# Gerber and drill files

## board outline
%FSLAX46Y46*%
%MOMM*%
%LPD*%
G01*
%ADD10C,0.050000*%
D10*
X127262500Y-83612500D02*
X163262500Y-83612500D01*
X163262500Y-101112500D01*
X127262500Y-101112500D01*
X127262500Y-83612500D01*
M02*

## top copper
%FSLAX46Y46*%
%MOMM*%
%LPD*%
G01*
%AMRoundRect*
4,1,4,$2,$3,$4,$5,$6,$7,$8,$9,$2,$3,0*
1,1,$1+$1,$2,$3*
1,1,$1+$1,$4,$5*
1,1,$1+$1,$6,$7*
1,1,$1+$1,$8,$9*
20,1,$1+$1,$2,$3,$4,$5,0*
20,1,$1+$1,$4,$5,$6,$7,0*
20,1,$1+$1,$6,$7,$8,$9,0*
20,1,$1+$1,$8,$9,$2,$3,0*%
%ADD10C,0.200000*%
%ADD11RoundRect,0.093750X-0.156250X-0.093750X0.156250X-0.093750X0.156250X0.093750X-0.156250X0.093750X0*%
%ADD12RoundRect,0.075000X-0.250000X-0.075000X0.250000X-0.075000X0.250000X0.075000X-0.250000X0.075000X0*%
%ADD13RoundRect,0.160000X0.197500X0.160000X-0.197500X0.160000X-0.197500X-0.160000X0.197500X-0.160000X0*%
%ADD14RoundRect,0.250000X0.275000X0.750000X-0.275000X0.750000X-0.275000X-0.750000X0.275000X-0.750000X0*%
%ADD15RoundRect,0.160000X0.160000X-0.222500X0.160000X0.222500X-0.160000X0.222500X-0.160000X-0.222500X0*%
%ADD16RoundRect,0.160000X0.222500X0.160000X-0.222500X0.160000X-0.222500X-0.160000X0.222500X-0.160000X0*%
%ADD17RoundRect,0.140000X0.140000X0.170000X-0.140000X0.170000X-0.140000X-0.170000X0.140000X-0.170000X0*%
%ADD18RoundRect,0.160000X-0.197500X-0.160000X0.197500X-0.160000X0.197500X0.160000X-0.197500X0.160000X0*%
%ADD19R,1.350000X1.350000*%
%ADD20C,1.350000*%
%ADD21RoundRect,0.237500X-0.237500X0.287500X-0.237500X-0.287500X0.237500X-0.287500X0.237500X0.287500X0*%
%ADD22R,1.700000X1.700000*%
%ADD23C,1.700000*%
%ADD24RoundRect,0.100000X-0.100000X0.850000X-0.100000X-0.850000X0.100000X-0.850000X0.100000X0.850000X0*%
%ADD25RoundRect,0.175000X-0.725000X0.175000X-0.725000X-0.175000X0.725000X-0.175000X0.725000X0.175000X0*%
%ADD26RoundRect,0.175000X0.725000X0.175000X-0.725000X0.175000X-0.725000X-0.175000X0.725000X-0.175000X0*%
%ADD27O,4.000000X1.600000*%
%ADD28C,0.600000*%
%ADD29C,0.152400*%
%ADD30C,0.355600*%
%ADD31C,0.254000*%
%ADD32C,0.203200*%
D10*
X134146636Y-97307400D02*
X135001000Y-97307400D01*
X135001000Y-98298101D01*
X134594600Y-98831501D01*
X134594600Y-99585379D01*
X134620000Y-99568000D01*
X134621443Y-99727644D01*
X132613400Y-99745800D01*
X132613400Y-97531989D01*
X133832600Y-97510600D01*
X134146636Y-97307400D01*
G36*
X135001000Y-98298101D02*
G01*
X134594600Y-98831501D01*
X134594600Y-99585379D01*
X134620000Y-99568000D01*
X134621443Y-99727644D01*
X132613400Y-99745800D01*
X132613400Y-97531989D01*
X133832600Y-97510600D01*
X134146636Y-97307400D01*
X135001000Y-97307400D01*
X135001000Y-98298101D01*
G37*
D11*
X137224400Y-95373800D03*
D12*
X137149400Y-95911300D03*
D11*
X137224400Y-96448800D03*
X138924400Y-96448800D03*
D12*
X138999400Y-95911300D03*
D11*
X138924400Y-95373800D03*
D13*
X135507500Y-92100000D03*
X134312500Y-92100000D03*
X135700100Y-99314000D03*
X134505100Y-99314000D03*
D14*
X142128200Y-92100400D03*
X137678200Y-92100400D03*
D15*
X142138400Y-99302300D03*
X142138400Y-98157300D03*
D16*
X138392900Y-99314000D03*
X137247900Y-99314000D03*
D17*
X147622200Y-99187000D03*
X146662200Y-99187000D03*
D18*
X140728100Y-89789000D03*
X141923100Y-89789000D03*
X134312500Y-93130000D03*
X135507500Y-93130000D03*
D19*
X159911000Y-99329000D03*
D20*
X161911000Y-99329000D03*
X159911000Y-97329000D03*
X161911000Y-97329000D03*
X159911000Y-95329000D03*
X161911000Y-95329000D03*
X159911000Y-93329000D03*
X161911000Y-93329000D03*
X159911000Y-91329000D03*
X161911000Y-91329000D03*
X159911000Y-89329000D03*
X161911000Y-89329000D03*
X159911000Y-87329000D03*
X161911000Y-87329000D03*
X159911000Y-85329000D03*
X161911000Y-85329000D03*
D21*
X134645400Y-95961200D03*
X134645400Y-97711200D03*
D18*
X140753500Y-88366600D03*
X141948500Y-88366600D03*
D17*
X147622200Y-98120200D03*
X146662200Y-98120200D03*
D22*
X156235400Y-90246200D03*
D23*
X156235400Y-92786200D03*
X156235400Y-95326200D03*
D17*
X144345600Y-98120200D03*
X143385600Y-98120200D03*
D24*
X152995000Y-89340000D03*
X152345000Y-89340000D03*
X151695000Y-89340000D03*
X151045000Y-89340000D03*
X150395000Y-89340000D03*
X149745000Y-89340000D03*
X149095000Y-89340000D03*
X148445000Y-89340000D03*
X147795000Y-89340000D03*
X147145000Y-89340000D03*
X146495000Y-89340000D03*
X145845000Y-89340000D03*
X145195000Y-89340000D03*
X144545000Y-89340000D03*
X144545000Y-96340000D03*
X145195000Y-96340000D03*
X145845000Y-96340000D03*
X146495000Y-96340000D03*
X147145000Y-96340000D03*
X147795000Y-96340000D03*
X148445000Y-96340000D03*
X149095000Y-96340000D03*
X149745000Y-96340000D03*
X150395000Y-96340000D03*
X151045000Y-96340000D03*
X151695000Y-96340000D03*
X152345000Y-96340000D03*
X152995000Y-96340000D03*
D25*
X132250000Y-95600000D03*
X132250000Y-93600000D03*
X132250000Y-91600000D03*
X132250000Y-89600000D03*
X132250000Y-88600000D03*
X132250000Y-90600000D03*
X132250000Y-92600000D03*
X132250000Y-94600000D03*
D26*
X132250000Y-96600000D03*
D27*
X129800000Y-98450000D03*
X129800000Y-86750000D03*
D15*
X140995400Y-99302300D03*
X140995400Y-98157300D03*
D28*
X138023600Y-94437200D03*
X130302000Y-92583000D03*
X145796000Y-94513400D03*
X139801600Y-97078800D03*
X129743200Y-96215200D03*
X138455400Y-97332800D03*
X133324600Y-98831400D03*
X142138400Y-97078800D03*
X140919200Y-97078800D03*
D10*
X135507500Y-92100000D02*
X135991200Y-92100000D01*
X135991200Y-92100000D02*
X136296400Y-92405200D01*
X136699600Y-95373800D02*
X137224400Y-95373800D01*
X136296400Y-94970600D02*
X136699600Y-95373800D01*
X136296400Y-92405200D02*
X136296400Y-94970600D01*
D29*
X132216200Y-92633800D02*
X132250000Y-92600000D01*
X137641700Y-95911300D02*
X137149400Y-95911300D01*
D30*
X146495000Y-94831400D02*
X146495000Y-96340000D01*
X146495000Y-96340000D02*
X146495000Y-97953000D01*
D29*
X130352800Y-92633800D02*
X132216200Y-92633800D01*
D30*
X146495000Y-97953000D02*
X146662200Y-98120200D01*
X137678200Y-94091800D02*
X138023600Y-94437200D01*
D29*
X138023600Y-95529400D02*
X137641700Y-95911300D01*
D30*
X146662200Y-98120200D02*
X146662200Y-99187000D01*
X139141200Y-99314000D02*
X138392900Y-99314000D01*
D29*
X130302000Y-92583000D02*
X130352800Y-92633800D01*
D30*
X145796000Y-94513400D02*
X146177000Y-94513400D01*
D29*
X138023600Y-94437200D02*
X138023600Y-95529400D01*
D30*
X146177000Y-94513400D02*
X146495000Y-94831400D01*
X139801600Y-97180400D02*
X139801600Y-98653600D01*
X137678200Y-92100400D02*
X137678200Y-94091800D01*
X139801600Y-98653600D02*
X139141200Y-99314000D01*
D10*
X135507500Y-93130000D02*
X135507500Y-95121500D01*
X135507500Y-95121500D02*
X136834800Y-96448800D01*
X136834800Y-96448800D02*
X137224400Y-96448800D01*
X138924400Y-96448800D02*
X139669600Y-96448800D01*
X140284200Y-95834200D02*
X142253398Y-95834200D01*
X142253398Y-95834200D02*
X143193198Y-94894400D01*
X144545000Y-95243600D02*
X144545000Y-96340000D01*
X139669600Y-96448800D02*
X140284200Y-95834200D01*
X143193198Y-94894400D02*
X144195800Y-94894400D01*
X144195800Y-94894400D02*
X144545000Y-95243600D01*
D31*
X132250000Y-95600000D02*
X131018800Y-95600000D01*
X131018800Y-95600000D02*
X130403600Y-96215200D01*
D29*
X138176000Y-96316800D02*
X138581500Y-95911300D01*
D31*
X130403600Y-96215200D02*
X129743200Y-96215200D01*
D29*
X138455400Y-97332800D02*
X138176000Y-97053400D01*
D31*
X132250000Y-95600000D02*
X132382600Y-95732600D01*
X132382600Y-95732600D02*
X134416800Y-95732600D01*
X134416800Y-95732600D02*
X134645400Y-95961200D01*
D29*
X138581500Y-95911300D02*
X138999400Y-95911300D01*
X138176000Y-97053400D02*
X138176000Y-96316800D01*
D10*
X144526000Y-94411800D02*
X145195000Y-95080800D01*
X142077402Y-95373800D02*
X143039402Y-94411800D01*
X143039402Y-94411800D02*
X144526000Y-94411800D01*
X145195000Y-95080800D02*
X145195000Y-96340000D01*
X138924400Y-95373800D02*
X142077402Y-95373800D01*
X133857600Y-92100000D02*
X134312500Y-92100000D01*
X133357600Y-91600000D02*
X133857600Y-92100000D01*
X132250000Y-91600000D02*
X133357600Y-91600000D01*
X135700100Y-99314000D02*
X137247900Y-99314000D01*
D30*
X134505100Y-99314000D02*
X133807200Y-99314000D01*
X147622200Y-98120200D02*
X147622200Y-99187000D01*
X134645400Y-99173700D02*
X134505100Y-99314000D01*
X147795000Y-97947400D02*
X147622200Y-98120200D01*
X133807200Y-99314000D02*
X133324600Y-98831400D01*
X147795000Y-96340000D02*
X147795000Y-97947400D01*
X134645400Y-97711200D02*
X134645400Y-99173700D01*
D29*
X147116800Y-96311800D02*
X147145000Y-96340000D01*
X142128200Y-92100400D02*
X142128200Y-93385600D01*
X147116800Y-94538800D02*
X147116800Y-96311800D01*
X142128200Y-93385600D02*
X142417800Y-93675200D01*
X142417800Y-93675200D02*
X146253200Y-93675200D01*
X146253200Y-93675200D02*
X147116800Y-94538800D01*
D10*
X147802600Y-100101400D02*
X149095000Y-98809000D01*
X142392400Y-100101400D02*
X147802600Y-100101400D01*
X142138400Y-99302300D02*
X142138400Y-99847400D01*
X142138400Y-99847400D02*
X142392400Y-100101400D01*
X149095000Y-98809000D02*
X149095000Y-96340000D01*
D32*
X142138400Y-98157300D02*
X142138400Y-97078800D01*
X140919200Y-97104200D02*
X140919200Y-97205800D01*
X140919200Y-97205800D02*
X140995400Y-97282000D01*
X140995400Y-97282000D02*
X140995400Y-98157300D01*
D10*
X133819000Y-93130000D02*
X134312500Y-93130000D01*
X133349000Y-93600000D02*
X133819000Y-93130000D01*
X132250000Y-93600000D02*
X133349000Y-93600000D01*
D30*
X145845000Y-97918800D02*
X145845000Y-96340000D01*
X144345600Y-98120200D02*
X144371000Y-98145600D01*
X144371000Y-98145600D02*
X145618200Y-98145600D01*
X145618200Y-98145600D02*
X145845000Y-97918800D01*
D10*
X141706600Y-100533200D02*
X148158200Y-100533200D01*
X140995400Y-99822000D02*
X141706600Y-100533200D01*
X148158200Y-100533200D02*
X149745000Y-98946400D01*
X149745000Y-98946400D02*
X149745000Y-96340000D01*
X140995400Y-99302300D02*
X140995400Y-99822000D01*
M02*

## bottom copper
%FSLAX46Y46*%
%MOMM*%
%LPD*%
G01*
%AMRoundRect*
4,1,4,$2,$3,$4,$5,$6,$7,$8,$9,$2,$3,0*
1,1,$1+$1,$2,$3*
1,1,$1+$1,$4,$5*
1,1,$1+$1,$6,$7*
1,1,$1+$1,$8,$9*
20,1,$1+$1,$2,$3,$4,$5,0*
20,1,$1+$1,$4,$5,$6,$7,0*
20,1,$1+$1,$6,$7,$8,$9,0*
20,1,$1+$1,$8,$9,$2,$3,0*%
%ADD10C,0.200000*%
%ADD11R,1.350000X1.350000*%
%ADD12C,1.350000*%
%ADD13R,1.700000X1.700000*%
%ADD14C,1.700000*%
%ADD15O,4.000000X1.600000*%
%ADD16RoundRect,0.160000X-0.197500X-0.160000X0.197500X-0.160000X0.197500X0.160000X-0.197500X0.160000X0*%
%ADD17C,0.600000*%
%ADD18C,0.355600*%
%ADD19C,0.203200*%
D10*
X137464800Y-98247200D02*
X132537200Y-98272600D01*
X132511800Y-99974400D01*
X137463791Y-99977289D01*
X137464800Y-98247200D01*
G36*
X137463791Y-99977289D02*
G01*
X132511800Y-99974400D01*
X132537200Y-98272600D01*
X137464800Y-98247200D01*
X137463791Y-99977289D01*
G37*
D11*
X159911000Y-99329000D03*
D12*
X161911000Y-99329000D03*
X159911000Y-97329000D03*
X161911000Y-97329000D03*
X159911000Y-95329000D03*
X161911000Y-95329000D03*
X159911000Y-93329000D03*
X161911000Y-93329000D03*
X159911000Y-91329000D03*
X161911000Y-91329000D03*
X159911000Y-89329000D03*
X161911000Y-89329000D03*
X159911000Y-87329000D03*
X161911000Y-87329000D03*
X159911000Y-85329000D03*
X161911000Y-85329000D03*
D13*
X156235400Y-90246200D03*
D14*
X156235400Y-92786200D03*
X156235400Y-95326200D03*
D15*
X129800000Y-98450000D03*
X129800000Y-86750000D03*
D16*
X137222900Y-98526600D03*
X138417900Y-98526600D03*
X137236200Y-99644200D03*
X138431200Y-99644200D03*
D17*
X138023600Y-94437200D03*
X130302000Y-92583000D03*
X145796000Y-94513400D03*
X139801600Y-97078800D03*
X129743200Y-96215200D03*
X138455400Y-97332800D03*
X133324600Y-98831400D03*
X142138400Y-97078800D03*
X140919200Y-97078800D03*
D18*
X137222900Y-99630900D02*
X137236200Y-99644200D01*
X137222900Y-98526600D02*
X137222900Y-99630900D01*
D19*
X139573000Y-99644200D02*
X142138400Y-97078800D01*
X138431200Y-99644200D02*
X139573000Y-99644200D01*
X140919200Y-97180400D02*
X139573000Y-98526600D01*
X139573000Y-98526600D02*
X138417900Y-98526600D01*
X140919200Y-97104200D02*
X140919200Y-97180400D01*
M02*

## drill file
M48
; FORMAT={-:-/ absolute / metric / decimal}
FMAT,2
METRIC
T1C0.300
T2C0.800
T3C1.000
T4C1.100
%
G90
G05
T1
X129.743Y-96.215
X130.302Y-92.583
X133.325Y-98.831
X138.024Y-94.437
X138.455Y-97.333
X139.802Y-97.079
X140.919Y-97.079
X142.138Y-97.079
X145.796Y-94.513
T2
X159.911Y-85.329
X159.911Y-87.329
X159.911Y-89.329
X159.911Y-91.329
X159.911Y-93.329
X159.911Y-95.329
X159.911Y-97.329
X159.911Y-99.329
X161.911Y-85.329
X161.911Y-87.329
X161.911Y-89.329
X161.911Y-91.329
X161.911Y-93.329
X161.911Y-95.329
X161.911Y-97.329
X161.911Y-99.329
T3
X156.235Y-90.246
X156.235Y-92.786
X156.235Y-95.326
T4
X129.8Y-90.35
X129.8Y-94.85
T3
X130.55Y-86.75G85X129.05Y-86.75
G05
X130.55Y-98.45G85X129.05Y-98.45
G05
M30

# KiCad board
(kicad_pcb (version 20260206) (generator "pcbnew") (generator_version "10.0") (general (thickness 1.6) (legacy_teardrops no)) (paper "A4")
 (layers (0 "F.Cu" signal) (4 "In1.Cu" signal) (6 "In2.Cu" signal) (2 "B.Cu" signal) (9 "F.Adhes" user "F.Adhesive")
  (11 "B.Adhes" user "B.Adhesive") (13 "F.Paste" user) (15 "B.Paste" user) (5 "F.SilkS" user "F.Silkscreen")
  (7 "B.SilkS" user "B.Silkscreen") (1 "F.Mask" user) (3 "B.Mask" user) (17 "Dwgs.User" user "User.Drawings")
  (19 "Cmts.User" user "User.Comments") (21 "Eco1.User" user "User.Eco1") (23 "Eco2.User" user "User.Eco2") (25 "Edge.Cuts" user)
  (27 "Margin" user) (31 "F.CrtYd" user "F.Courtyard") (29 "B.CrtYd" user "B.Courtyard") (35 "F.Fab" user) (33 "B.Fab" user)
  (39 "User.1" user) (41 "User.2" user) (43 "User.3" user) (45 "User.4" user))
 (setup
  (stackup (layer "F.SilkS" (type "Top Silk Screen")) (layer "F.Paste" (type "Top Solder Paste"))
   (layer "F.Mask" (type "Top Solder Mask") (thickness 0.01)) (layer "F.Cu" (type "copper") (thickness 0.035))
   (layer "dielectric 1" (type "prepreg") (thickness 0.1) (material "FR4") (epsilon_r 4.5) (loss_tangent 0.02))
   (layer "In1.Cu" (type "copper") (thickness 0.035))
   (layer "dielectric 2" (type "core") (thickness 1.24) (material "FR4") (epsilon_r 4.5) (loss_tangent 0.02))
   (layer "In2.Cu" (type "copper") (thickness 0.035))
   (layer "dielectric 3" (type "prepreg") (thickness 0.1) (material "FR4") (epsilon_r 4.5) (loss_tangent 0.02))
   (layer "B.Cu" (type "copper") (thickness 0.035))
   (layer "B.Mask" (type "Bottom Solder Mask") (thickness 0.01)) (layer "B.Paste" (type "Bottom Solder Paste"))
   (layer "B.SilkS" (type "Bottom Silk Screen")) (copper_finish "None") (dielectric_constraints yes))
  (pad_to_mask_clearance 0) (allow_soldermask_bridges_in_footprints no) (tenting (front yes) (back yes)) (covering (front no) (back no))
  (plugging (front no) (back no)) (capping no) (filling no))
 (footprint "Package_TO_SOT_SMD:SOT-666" (layer "F.Cu") (at 138.0744 95.9113)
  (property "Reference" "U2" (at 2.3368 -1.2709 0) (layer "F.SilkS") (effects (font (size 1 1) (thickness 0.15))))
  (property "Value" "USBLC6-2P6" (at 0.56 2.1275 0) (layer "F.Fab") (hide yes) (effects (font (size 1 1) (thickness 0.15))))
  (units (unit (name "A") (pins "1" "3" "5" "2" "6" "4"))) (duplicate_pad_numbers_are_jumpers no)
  (pad "1" smd roundrect (at -0.85 -0.5375) (size 0.5 0.375) (layers "F.Cu" "F.Mask" "F.Paste") (roundrect_rratio 0.25) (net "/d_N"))
  (pad "2" smd roundrect (at -0.925 0) (size 0.65 0.3) (layers "F.Cu" "F.Mask" "F.Paste") (roundrect_rratio 0.25) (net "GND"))
  (pad "3" smd roundrect (at -0.85 0.5375) (size 0.5 0.375) (layers "F.Cu" "F.Mask" "F.Paste") (roundrect_rratio 0.25) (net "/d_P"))
  (pad "4" smd roundrect (at 0.85 0.5375) (size 0.5 0.375) (layers "F.Cu" "F.Mask" "F.Paste") (roundrect_rratio 0.25) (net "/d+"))
  (pad "5" smd roundrect (at 0.925 0) (size 0.65 0.3) (layers "F.Cu" "F.Mask" "F.Paste") (roundrect_rratio 0.25) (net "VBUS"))
  (pad "6" smd roundrect (at 0.85 -0.5375) (size 0.5 0.375) (layers "F.Cu" "F.Mask" "F.Paste") (roundrect_rratio 0.25) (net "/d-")))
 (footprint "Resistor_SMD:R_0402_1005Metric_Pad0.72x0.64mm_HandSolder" (layer "F.Cu") (at 134.91 92.1 180)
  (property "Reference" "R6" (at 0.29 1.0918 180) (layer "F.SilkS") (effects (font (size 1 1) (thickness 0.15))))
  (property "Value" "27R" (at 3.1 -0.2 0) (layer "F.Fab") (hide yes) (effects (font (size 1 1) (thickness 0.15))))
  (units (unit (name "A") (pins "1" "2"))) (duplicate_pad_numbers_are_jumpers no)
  (pad "1" smd roundrect (at -0.5975 0 180) (size 0.715 0.64) (layers "F.Cu" "F.Mask" "F.Paste") (roundrect_rratio 0.25) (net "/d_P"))
  (pad "2" smd roundrect (at 0.5975 0 180) (size 0.715 0.64) (layers "F.Cu" "F.Mask" "F.Paste") (roundrect_rratio 0.25) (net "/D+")))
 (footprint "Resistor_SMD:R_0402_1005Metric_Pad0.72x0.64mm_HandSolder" (layer "F.Cu") (at 135.1026 99.314 180)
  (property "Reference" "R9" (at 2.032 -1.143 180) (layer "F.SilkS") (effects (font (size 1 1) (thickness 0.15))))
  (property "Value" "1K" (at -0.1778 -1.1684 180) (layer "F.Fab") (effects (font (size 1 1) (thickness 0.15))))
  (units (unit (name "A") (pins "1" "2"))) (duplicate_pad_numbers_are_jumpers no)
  (pad "1" smd roundrect (at -0.5975 0 180) (size 0.715 0.64) (layers "F.Cu" "F.Mask" "F.Paste") (roundrect_rratio 0.25) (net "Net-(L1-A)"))
  (pad "2" smd roundrect (at 0.5975 0 180) (size 0.715 0.64) (layers "F.Cu" "F.Mask" "F.Paste") (roundrect_rratio 0.25) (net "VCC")))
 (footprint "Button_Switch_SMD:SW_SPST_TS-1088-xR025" (layer "F.Cu") (at 139.9032 92.1004 180)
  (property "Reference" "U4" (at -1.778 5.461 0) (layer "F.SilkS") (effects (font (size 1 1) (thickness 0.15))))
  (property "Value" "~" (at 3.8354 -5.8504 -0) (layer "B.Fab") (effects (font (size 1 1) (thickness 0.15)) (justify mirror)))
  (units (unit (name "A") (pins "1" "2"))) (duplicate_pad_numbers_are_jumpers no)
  (pad "1" smd roundrect (at -2.225 0 180) (size 1.05 2) (layers "F.Cu" "F.Mask" "F.Paste") (roundrect_rratio 0.2380952381) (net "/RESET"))
  (pad "2" smd roundrect (at 2.225 0 180) (size 1.05 2) (layers "F.Cu" "F.Mask" "F.Paste") (roundrect_rratio 0.2380952381) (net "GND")))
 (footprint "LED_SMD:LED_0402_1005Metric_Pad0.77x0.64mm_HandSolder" (layer "F.Cu") (at 142.1384 98.7298 90)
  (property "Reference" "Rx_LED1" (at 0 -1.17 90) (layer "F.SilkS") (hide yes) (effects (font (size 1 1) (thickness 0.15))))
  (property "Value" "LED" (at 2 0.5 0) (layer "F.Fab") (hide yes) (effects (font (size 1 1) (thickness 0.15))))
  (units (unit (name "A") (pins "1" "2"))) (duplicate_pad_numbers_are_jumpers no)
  (pad "1" smd roundrect (at -0.5725 0 90) (size 0.765 0.64) (layers "F.Cu" "F.Mask" "F.Paste") (roundrect_rratio 0.25)
   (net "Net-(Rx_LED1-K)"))
  (pad "2" smd roundrect (at 0.5725 0 90) (size 0.765 0.64) (layers "F.Cu" "F.Mask" "F.Paste") (roundrect_rratio 0.25) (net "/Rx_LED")))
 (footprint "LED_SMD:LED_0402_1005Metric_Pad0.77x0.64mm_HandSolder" (layer "F.Cu") (at 137.8204 99.314 180)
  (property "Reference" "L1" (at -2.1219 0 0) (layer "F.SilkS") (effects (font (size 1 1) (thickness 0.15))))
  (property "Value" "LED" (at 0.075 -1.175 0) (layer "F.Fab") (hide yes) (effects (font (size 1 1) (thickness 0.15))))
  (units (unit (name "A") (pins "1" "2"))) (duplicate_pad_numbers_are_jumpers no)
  (pad "1" smd roundrect (at -0.5725 0 180) (size 0.765 0.64) (layers "F.Cu" "F.Mask" "F.Paste") (roundrect_rratio 0.25) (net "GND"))
  (pad "2" smd roundrect (at 0.5725 0 180) (size 0.765 0.64) (layers "F.Cu" "F.Mask" "F.Paste") (roundrect_rratio 0.25) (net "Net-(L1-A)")))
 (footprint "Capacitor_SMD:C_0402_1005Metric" (layer "F.Cu") (at 147.1422 99.187 180)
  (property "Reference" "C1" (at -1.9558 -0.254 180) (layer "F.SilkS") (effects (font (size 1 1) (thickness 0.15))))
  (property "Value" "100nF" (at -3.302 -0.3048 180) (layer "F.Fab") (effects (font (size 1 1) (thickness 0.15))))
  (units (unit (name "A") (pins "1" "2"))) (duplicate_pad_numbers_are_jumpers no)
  (pad "1" smd roundrect (at -0.48 0 180) (size 0.56 0.62) (layers "F.Cu" "F.Mask" "F.Paste") (roundrect_rratio 0.25) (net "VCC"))
  (pad "2" smd roundrect (at 0.48 0 180) (size 0.56 0.62) (layers "F.Cu" "F.Mask" "F.Paste") (roundrect_rratio 0.25) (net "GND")))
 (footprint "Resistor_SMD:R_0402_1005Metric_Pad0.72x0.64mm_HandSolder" (layer "F.Cu") (at 141.3256 89.789)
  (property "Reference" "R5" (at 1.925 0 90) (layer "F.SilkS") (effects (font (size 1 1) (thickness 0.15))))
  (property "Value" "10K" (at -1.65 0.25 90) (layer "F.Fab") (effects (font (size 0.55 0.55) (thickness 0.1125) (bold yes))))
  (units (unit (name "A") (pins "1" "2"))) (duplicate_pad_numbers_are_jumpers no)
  (pad "1" smd roundrect (at -0.5975 0) (size 0.715 0.64) (layers "F.Cu" "F.Mask" "F.Paste") (roundrect_rratio 0.25) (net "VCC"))
  (pad "2" smd roundrect (at 0.5975 0) (size 0.715 0.64) (layers "F.Cu" "F.Mask" "F.Paste") (roundrect_rratio 0.25) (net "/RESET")))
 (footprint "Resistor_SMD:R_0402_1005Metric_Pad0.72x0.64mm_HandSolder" (layer "F.Cu") (at 134.91 93.13)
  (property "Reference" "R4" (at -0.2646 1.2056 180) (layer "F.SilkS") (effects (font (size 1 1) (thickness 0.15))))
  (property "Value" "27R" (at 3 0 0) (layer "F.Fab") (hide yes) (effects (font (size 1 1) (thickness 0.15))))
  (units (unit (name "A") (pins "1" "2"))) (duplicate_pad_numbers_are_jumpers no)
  (pad "1" smd roundrect (at -0.5975 0) (size 0.715 0.64) (layers "F.Cu" "F.Mask" "F.Paste") (roundrect_rratio 0.25) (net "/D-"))
  (pad "2" smd roundrect (at 0.5975 0) (size 0.715 0.64) (layers "F.Cu" "F.Mask" "F.Paste") (roundrect_rratio 0.25) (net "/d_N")))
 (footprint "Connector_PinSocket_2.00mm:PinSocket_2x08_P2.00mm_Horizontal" (layer "F.Cu") (at 159.911 99.329 180)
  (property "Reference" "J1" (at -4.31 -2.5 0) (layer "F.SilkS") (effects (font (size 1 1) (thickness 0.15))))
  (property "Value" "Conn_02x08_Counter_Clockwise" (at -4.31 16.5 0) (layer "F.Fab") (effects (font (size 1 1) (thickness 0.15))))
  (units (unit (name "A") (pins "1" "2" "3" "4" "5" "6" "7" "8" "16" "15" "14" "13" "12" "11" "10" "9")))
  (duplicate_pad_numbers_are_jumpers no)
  (pad "1" thru_hole rect (at 0 0 180) (size 1.35 1.35) (drill 0.8) (layers "*.Cu" "*.Mask") (remove_unused_layers no)
   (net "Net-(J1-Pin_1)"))
  (pad "2" thru_hole circle (at -2 0 180) (size 1.35 1.35) (drill 0.8) (layers "*.Cu" "*.Mask") (remove_unused_layers no)
   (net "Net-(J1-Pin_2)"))
  (pad "3" thru_hole circle (at 0 2 180) (size 1.35 1.35) (drill 0.8) (layers "*.Cu" "*.Mask") (remove_unused_layers no)
   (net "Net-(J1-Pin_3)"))
  (pad "4" thru_hole circle (at -2 2 180) (size 1.35 1.35) (drill 0.8) (layers "*.Cu" "*.Mask") (remove_unused_layers no)
   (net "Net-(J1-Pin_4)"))
  (pad "5" thru_hole circle (at 0 4 180) (size 1.35 1.35) (drill 0.8) (layers "*.Cu" "*.Mask") (remove_unused_layers no)
   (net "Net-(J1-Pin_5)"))
  (pad "6" thru_hole circle (at -2 4 180) (size 1.35 1.35) (drill 0.8) (layers "*.Cu" "*.Mask") (remove_unused_layers no)
   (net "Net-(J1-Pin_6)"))
  (pad "7" thru_hole circle (at 0 6 180) (size 1.35 1.35) (drill 0.8) (layers "*.Cu" "*.Mask") (remove_unused_layers no)
   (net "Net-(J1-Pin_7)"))
  (pad "8" thru_hole circle (at -2 6 180) (size 1.35 1.35) (drill 0.8) (layers "*.Cu" "*.Mask") (remove_unused_layers no)
   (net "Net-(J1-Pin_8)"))
  (pad "9" thru_hole circle (at 0 8 180) (size 1.35 1.35) (drill 0.8) (layers "*.Cu" "*.Mask") (remove_unused_layers no)
   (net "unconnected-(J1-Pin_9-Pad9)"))
  (pad "10" thru_hole circle (at -2 8 180) (size 1.35 1.35) (drill 0.8) (layers "*.Cu" "*.Mask") (remove_unused_layers no)
   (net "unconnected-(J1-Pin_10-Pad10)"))
  (pad "11" thru_hole circle (at 0 10 180) (size 1.35 1.35) (drill 0.8) (layers "*.Cu" "*.Mask") (remove_unused_layers no)
   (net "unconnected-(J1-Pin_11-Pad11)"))
  (pad "12" thru_hole circle (at -2 10 180) (size 1.35 1.35) (drill 0.8) (layers "*.Cu" "*.Mask") (remove_unused_layers no)
   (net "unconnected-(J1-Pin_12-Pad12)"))
  (pad "13" thru_hole circle (at 0 12 180) (size 1.35 1.35) (drill 0.8) (layers "*.Cu" "*.Mask") (remove_unused_layers no)
   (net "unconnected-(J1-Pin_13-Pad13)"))
  (pad "14" thru_hole circle (at -2 12 180) (size 1.35 1.35) (drill 0.8) (layers "*.Cu" "*.Mask") (remove_unused_layers no)
   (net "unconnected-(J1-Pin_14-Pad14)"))
  (pad "15" thru_hole circle (at 0 14 180) (size 1.35 1.35) (drill 0.8) (layers "*.Cu" "*.Mask") (remove_unused_layers no)
   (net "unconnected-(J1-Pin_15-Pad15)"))
  (pad "16" thru_hole circle (at -2 14 180) (size 1.35 1.35) (drill 0.8) (layers "*.Cu" "*.Mask") (remove_unused_layers no)
   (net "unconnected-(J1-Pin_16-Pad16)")))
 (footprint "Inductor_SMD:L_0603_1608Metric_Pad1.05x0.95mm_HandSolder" (layer "F.Cu") (at 134.6454 96.8362 -90)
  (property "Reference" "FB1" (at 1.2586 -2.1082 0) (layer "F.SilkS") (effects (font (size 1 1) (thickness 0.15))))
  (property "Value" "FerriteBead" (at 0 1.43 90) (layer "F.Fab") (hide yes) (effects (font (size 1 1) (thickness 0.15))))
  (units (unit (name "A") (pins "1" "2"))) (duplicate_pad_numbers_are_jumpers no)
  (pad "1" smd roundrect (at -0.875 0 270) (size 1.05 0.95) (layers "F.Cu" "F.Mask" "F.Paste") (roundrect_rratio 0.25) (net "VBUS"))
  (pad "2" smd roundrect (at 0.875 0 270) (size 1.05 0.95) (layers "F.Cu" "F.Mask" "F.Paste") (roundrect_rratio 0.25) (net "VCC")))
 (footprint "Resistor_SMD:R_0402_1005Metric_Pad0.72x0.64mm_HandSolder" (layer "F.Cu") (at 141.351 88.3666)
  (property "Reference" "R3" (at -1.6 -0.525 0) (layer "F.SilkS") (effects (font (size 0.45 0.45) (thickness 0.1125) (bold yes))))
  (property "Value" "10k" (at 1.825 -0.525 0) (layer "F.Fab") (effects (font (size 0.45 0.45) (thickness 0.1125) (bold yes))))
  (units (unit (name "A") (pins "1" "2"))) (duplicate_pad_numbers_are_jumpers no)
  (pad "1" smd roundrect (at -0.5975 0) (size 0.715 0.64) (layers "F.Cu" "F.Mask" "F.Paste") (roundrect_rratio 0.25) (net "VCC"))
  (pad "2" smd roundrect (at 0.5975 0) (size 0.715 0.64) (layers "F.Cu" "F.Mask" "F.Paste") (roundrect_rratio 0.25) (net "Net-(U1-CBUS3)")))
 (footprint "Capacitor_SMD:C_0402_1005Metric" (layer "F.Cu") (at 147.1422 98.1202 180)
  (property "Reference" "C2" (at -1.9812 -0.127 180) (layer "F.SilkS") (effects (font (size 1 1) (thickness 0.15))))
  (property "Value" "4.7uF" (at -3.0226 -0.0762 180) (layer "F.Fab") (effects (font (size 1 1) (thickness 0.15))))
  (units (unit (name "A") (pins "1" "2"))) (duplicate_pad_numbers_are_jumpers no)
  (pad "1" smd roundrect (at -0.48 0 180) (size 0.56 0.62) (layers "F.Cu" "F.Mask" "F.Paste") (roundrect_rratio 0.25) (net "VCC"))
  (pad "2" smd roundrect (at 0.48 0 180) (size 0.56 0.62) (layers "F.Cu" "F.Mask" "F.Paste") (roundrect_rratio 0.25) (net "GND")))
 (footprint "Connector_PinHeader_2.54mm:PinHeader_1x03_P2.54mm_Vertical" (layer "F.Cu") (at 156.2354 90.2462)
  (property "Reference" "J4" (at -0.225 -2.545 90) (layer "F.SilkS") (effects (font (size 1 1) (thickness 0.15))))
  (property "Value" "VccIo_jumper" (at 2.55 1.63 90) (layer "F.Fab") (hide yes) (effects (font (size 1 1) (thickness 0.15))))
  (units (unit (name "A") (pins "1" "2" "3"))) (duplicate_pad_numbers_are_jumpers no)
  (pad "1" thru_hole rect (at 0 0) (size 1.7 1.7) (drill 1) (layers "*.Cu" "*.Mask") (remove_unused_layers no) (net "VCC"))
  (pad "2" thru_hole circle (at 0 2.54) (size 1.7 1.7) (drill 1) (layers "*.Cu" "*.Mask") (remove_unused_layers no) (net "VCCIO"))
  (pad "3" thru_hole circle (at 0 5.08) (size 1.7 1.7) (drill 1) (layers "*.Cu" "*.Mask") (remove_unused_layers no) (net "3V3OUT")))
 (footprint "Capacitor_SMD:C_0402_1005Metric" (layer "F.Cu") (at 143.8656 98.1202 180)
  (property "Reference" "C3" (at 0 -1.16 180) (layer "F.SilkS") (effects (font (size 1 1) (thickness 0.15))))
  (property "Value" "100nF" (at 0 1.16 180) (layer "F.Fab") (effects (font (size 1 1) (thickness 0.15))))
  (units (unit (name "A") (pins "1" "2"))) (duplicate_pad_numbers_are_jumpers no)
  (pad "1" smd roundrect (at -0.48 0 180) (size 0.56 0.62) (layers "F.Cu" "F.Mask" "F.Paste") (roundrect_rratio 0.25) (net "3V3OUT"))
  (pad "2" smd roundrect (at 0.48 0 180) (size 0.56 0.62) (layers "F.Cu" "F.Mask" "F.Paste") (roundrect_rratio 0.25) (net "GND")))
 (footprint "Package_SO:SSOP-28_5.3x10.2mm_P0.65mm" (layer "F.Cu") (at 148.77 92.84 -90)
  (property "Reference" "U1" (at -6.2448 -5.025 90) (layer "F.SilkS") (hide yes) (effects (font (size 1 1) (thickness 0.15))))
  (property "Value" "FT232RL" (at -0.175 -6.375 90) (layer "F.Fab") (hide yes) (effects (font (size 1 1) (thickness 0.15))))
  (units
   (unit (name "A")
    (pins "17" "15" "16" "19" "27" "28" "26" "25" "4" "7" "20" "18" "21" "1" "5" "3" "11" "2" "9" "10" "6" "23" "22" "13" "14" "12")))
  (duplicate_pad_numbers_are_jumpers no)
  (pad "1" smd roundrect (at -3.5 -4.225 270) (size 1.9 0.4) (layers "F.Cu" "F.Mask" "F.Paste") (roundrect_rratio 0.25)
   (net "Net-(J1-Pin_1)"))
  (pad "2" smd roundrect (at -3.5 -3.575 270) (size 1.9 0.4) (layers "F.Cu" "F.Mask" "F.Paste") (roundrect_rratio 0.25)
   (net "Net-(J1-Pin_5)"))
  (pad "3" smd roundrect (at -3.5 -2.925 270) (size 1.9 0.4) (layers "F.Cu" "F.Mask" "F.Paste") (roundrect_rratio 0.25)
   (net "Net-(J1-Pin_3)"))
  (pad "4" smd roundrect (at -3.5 -2.275 270) (size 1.9 0.4) (layers "F.Cu" "F.Mask" "F.Paste") (roundrect_rratio 0.25) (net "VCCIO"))
  (pad "5" smd roundrect (at -3.5 -1.625 270) (size 1.9 0.4) (layers "F.Cu" "F.Mask" "F.Paste") (roundrect_rratio 0.25)
   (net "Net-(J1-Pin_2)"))
  (pad "6" smd roundrect (at -3.5 -0.975 270) (size 1.9 0.4) (layers "F.Cu" "F.Mask" "F.Paste") (roundrect_rratio 0.25)
   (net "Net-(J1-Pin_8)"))
  (pad "7" smd roundrect (at -3.5 -0.325 270) (size 1.9 0.4) (layers "F.Cu" "F.Mask" "F.Paste") (roundrect_rratio 0.25) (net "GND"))
  (pad "8" smd roundrect (at -3.5 0.325 270) (size 1.9 0.4) (layers "F.Cu" "F.Mask" "F.Paste") (roundrect_rratio 0.25))
  (pad "9" smd roundrect (at -3.5 0.975 270) (size 1.9 0.4) (layers "F.Cu" "F.Mask" "F.Paste") (roundrect_rratio 0.25)
   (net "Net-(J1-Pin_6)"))
  (pad "10" smd roundrect (at -3.5 1.625 270) (size 1.9 0.4) (layers "F.Cu" "F.Mask" "F.Paste") (roundrect_rratio 0.25)
   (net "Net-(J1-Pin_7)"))
  (pad "11" smd roundrect (at -3.5 2.275 270) (size 1.9 0.4) (layers "F.Cu" "F.Mask" "F.Paste") (roundrect_rratio 0.25)
   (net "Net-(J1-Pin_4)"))
  (pad "12" smd roundrect (at -3.5 2.925 270) (size 1.9 0.4) (layers "F.Cu" "F.Mask" "F.Paste") (roundrect_rratio 0.25)
   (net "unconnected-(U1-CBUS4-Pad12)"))
  (pad "13" smd roundrect (at -3.5 3.575 270) (size 1.9 0.4) (layers "F.Cu" "F.Mask" "F.Paste") (roundrect_rratio 0.25)
   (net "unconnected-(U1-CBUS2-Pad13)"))
  (pad "14" smd roundrect (at -3.5 4.225 270) (size 1.9 0.4) (layers "F.Cu" "F.Mask" "F.Paste") (roundrect_rratio 0.25)
   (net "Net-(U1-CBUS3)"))
  (pad "15" smd roundrect (at 3.5 4.225 270) (size 1.9 0.4) (layers "F.Cu" "F.Mask" "F.Paste") (roundrect_rratio 0.25) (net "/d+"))
  (pad "16" smd roundrect (at 3.5 3.575 270) (size 1.9 0.4) (layers "F.Cu" "F.Mask" "F.Paste") (roundrect_rratio 0.25) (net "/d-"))
  (pad "17" smd roundrect (at 3.5 2.925 270) (size 1.9 0.4) (layers "F.Cu" "F.Mask" "F.Paste") (roundrect_rratio 0.25) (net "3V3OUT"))
  (pad "18" smd roundrect (at 3.5 2.275 270) (size 1.9 0.4) (layers "F.Cu" "F.Mask" "F.Paste") (roundrect_rratio 0.25) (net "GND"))
  (pad "19" smd roundrect (at 3.5 1.625 270) (size 1.9 0.4) (layers "F.Cu" "F.Mask" "F.Paste") (roundrect_rratio 0.25) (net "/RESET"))
  (pad "20" smd roundrect (at 3.5 0.975 270) (size 1.9 0.4) (layers "F.Cu" "F.Mask" "F.Paste") (roundrect_rratio 0.25) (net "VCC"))
  (pad "21" smd roundrect (at 3.5 0.325 270) (size 1.9 0.4) (layers "F.Cu" "F.Mask" "F.Paste") (roundrect_rratio 0.25) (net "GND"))
  (pad "22" smd roundrect (at 3.5 -0.325 270) (size 1.9 0.4) (layers "F.Cu" "F.Mask" "F.Paste") (roundrect_rratio 0.25)
   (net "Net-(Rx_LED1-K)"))
  (pad "23" smd roundrect (at 3.5 -0.975 270) (size 1.9 0.4) (layers "F.Cu" "F.Mask" "F.Paste") (roundrect_rratio 0.25)
   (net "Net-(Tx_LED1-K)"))
  (pad "24" smd roundrect (at 3.5 -1.625 270) (size 1.9 0.4) (layers "F.Cu" "F.Mask" "F.Paste") (roundrect_rratio 0.25))
  (pad "25" smd roundrect (at 3.5 -2.275 270) (size 1.9 0.4) (layers "F.Cu" "F.Mask" "F.Paste") (roundrect_rratio 0.25) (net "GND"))
  (pad "26" smd roundrect (at 3.5 -2.925 270) (size 1.9 0.4) (layers "F.Cu" "F.Mask" "F.Paste") (roundrect_rratio 0.25) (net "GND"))
  (pad "27" smd roundrect (at 3.5 -3.575 270) (size 1.9 0.4) (layers "F.Cu" "F.Mask" "F.Paste") (roundrect_rratio 0.25)
   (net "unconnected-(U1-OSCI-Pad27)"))
  (pad "28" smd roundrect (at 3.5 -4.225 270) (size 1.9 0.4) (layers "F.Cu" "F.Mask" "F.Paste") (roundrect_rratio 0.25)
   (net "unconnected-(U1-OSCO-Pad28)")))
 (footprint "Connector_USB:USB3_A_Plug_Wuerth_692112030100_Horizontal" (layer "F.Cu") (at 121.4 92.6 180)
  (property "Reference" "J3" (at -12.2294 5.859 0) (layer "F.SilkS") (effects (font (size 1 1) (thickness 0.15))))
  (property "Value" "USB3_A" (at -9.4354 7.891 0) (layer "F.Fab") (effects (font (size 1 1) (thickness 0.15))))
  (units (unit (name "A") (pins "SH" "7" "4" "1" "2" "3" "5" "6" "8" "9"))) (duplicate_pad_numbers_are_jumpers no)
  (pad "" np_thru_hole circle (at -8.4 -2.25 270) (size 1.1 1.1) (drill 1.1) (layers "*.Cu" "*.Mask"))
  (pad "" np_thru_hole circle (at -8.4 2.25 270) (size 1.1 1.1) (drill 1.1) (layers "*.Cu" "*.Mask"))
  (pad "1" smd roundrect (at -10.85 -3 270) (size 0.7 1.8) (layers "F.Cu" "F.Mask" "F.Paste") (roundrect_rratio 0.25) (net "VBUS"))
  (pad "2" smd roundrect (at -10.85 -1 270) (size 0.7 1.8) (layers "F.Cu" "F.Mask" "F.Paste") (roundrect_rratio 0.25) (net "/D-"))
  (pad "3" smd roundrect (at -10.85 1 270) (size 0.7 1.8) (layers "F.Cu" "F.Mask" "F.Paste") (roundrect_rratio 0.25) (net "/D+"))
  (pad "4" smd roundrect (at -10.85 3 270) (size 0.7 1.8) (layers "F.Cu" "F.Mask" "F.Paste") (roundrect_rratio 0.25) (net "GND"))
  (pad "5" smd roundrect (at -10.85 4 270) (size 0.7 1.8) (layers "F.Cu" "F.Mask" "F.Paste") (roundrect_rratio 0.25)
   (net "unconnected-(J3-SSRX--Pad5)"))
  (pad "6" smd roundrect (at -10.85 2 270) (size 0.7 1.8) (layers "F.Cu" "F.Mask" "F.Paste") (roundrect_rratio 0.25)
   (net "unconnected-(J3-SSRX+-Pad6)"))
  (pad "7" smd roundrect (at -10.85 0 270) (size 0.7 1.8) (layers "F.Cu" "F.Mask" "F.Paste") (roundrect_rratio 0.25) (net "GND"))
  (pad "8" smd roundrect (at -10.85 -2 270) (size 0.7 1.8) (layers "F.Cu" "F.Mask" "F.Paste") (roundrect_rratio 0.25)
   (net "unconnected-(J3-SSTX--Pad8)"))
  (pad "9" smd roundrect (at -10.85 -4 180) (size 1.8 0.7) (layers "F.Cu" "F.Mask" "F.Paste") (roundrect_rratio 0.25)
   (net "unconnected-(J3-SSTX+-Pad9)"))
  (pad "SH" thru_hole oval (at -8.4 -5.85 270) (size 1.6 4) (drill oval 1 2.5) (layers "*.Cu" "*.Mask") (remove_unused_layers no)
   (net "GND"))
  (pad "SH" thru_hole oval (at -8.4 5.85 270) (size 1.6 4) (drill oval 1 2.5) (layers "*.Cu" "*.Mask") (remove_unused_layers no) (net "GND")))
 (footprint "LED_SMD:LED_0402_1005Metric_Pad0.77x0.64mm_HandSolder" (layer "F.Cu") (at 140.9954 98.7298 90)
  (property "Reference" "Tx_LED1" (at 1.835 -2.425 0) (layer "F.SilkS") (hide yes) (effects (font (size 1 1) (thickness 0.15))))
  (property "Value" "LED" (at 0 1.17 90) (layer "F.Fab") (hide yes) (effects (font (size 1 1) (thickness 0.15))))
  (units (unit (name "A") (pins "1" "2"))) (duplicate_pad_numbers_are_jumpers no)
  (pad "1" smd roundrect (at -0.5725 0 90) (size 0.765 0.64) (layers "F.Cu" "F.Mask" "F.Paste") (roundrect_rratio 0.25)
   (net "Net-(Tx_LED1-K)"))
  (pad "2" smd roundrect (at 0.5725 0 90) (size 0.765 0.64) (layers "F.Cu" "F.Mask" "F.Paste") (roundrect_rratio 0.25) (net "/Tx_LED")))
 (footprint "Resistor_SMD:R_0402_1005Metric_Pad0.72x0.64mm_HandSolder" (layer "B.Cu") (at 137.8204 98.5266)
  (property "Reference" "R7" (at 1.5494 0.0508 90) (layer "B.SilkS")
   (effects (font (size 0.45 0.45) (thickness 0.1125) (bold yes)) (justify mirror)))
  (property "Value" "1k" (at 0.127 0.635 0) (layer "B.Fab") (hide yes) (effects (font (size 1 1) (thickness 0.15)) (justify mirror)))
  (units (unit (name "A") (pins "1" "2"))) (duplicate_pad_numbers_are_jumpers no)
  (pad "1" smd roundrect (at -0.5975 0) (size 0.715 0.64) (layers "B.Cu" "B.Mask" "B.Paste") (roundrect_rratio 0.25) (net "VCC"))
  (pad "2" smd roundrect (at 0.5975 0) (size 0.715 0.64) (layers "B.Cu" "B.Mask" "B.Paste") (roundrect_rratio 0.25) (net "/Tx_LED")))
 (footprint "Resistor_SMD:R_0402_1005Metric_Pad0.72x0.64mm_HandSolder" (layer "B.Cu") (at 137.8337 99.6442)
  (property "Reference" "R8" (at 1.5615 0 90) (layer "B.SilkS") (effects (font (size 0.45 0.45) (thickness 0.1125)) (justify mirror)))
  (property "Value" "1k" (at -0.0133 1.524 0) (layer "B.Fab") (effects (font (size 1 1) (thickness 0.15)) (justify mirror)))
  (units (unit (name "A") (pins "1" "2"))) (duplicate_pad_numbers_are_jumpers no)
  (pad "1" smd roundrect (at -0.5975 0) (size 0.715 0.64) (layers "B.Cu" "B.Mask" "B.Paste") (roundrect_rratio 0.25) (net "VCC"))
  (pad "2" smd roundrect (at 0.5975 0) (size 0.715 0.64) (layers "B.Cu" "B.Mask" "B.Paste") (roundrect_rratio 0.25) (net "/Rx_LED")))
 (gr_poly
  (pts (xy 134.146636 97.3074) (xy 135.001 97.3074) (xy 135.001 98.298101) (xy 134.5946 98.831501) (xy 134.5946 99.585379)
   (xy 134.62 99.568) (xy 134.621443 99.727644) (xy 132.6134 99.7458) (xy 132.6134 97.531989) (xy 133.8326 97.5106))
  (stroke (width 0.2) (type solid)) (fill yes) (layer "F.Cu") (net "VCC"))
 (gr_poly
  (pts (xy 137.4648 98.2472) (xy 132.5372 98.2726) (xy 132.5118 99.9744) (xy 137.463791 99.977289)) (stroke (width 0.2) (type solid))
  (fill yes) (layer "B.Cu") (net "VCC"))
 (gr_rect (start 127.2625 83.6125) (end 163.2625 101.1125) (stroke (width 0.05) (type solid)) (fill no) (layer "Edge.Cuts"))
 (segment (start 135.5075 92.1) (end 135.9912 92.1) (width 0.2) (layer "F.Cu") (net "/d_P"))
 (segment (start 135.9912 92.1) (end 136.2964 92.4052) (width 0.2) (layer "F.Cu") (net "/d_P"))
 (segment (start 136.6996 95.3738) (end 137.2244 95.3738) (width 0.2) (layer "F.Cu") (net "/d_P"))
 (segment (start 136.2964 94.9706) (end 136.6996 95.3738) (width 0.2) (layer "F.Cu") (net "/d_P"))
 (segment (start 136.2964 92.4052) (end 136.2964 94.9706) (width 0.2) (layer "F.Cu") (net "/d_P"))
 (segment (start 132.2162 92.6338) (end 132.25 92.6) (width 0.1524) (layer "F.Cu") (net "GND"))
 (segment (start 137.6417 95.9113) (end 137.1494 95.9113) (width 0.1524) (layer "F.Cu") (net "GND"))
 (segment (start 146.495 94.8314) (end 146.495 96.34) (width 0.3556) (layer "F.Cu") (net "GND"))
 (segment (start 146.495 96.34) (end 146.495 97.953) (width 0.3556) (layer "F.Cu") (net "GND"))
 (segment (start 130.3528 92.6338) (end 132.2162 92.6338) (width 0.1524) (layer "F.Cu") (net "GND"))
 (segment (start 146.495 97.953) (end 146.6622 98.1202) (width 0.3556) (layer "F.Cu") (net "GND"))
 (segment (start 137.6782 94.0918) (end 138.0236 94.4372) (width 0.3556) (layer "F.Cu") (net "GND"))
 (segment (start 138.0236 95.5294) (end 137.6417 95.9113) (width 0.1524) (layer "F.Cu") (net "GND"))
 (segment (start 146.6622 98.1202) (end 146.6622 99.187) (width 0.3556) (layer "F.Cu") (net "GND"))
 (segment (start 139.1412 99.314) (end 138.3929 99.314) (width 0.3556) (layer "F.Cu") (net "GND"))
 (segment (start 130.302 92.583) (end 130.3528 92.6338) (width 0.1524) (layer "F.Cu") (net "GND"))
 (segment (start 145.796 94.5134) (end 146.177 94.5134) (width 0.3556) (layer "F.Cu") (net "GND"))
 (segment (start 138.0236 94.4372) (end 138.0236 95.5294) (width 0.1524) (layer "F.Cu") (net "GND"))
 (segment (start 146.177 94.5134) (end 146.495 94.8314) (width 0.3556) (layer "F.Cu") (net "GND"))
 (segment (start 139.8016 97.1804) (end 139.8016 98.6536) (width 0.3556) (layer "F.Cu") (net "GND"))
 (segment (start 137.6782 92.1004) (end 137.6782 94.0918) (width 0.3556) (layer "F.Cu") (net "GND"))
 (segment (start 139.8016 98.6536) (end 139.1412 99.314) (width 0.3556) (layer "F.Cu") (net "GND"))
 (via (at 138.0236 94.4372) (size 0.6) (drill 0.3) (layers "F.Cu" "B.Cu") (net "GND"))
 (via (at 130.302 92.583) (size 0.6) (drill 0.3) (layers "F.Cu" "B.Cu") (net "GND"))
 (via (at 145.796 94.5134) (size 0.6) (drill 0.3) (layers "F.Cu" "B.Cu") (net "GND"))
 (via (at 139.8016 97.0788) (size 0.6) (drill 0.3) (layers "F.Cu" "B.Cu") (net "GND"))
 (segment (start 135.5075 93.13) (end 135.5075 95.1215) (width 0.2) (layer "F.Cu") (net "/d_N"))
 (segment (start 135.5075 95.1215) (end 136.8348 96.4488) (width 0.2) (layer "F.Cu") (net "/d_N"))
 (segment (start 136.8348 96.4488) (end 137.2244 96.4488) (width 0.2) (layer "F.Cu") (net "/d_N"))
 (segment (start 138.9244 96.4488) (end 139.6696 96.4488) (width 0.2) (layer "F.Cu") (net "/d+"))
 (segment (start 140.2842 95.8342) (end 142.253398 95.8342) (width 0.2) (layer "F.Cu") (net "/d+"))
 (segment (start 142.253398 95.8342) (end 143.193198 94.8944) (width 0.2) (layer "F.Cu") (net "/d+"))
 (segment (start 144.545 95.2436) (end 144.545 96.34) (width 0.2) (layer "F.Cu") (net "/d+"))
 (segment (start 139.6696 96.4488) (end 140.2842 95.8342) (width 0.2) (layer "F.Cu") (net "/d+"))
 (segment (start 143.193198 94.8944) (end 144.1958 94.8944) (width 0.2) (layer "F.Cu") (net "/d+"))
 (segment (start 144.1958 94.8944) (end 144.545 95.2436) (width 0.2) (layer "F.Cu") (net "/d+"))
 (segment (start 132.25 95.6) (end 131.0188 95.6) (width 0.254) (layer "F.Cu") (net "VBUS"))
 (segment (start 131.0188 95.6) (end 130.4036 96.2152) (width 0.254) (layer "F.Cu") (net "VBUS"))
 (segment (start 138.176 96.3168) (end 138.5815 95.9113) (width 0.1524) (layer "F.Cu") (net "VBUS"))
 (segment (start 130.4036 96.2152) (end 129.7432 96.2152) (width 0.254) (layer "F.Cu") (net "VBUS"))
 (segment (start 138.4554 97.3328) (end 138.176 97.0534) (width 0.1524) (layer "F.Cu") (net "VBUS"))
 (segment (start 132.25 95.6) (end 132.3826 95.7326) (width 0.254) (layer "F.Cu") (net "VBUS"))
 (segment (start 132.3826 95.7326) (end 134.4168 95.7326) (width 0.254) (layer "F.Cu") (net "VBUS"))
 (segment (start 134.4168 95.7326) (end 134.6454 95.9612) (width 0.254) (layer "F.Cu") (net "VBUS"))
 (segment (start 138.5815 95.9113) (end 138.9994 95.9113) (width 0.1524) (layer "F.Cu") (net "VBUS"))
 (segment (start 138.176 97.0534) (end 138.176 96.3168) (width 0.1524) (layer "F.Cu") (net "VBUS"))
 (via (at 129.7432 96.2152) (size 0.6) (drill 0.3) (layers "F.Cu" "B.Cu") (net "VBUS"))
 (via (at 138.4554 97.3328) (size 0.6) (drill 0.3) (layers "F.Cu" "B.Cu") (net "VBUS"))
 (segment (start 144.526 94.4118) (end 145.195 95.0808) (width 0.2) (layer "F.Cu") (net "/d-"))
 (segment (start 142.077402 95.3738) (end 143.039402 94.4118) (width 0.2) (layer "F.Cu") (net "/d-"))
 (segment (start 143.039402 94.4118) (end 144.526 94.4118) (width 0.2) (layer "F.Cu") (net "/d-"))
 (segment (start 145.195 95.0808) (end 145.195 96.34) (width 0.2) (layer "F.Cu") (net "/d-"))
 (segment (start 138.9244 95.3738) (end 142.077402 95.3738) (width 0.2) (layer "F.Cu") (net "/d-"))
 (segment (start 133.8576 92.1) (end 134.3125 92.1) (width 0.2) (layer "F.Cu") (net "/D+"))
 (segment (start 133.3576 91.6) (end 133.8576 92.1) (width 0.2) (layer "F.Cu") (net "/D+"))
 (segment (start 132.25 91.6) (end 133.3576 91.6) (width 0.2) (layer "F.Cu") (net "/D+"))
 (segment (start 135.7001 99.314) (end 137.2479 99.314) (width 0.2) (layer "F.Cu") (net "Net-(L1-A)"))
 (segment (start 134.5051 99.314) (end 133.8072 99.314) (width 0.3556) (layer "F.Cu") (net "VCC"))
 (segment (start 147.6222 98.1202) (end 147.6222 99.187) (width 0.3556) (layer "F.Cu") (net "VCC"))
 (segment (start 134.6454 99.1737) (end 134.5051 99.314) (width 0.3556) (layer "F.Cu") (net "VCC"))
 (segment (start 147.795 97.9474) (end 147.6222 98.1202) (width 0.3556) (layer "F.Cu") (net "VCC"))
 (segment (start 133.8072 99.314) (end 133.3246 98.8314) (width 0.3556) (layer "F.Cu") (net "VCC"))
 (segment (start 147.795 96.34) (end 147.795 97.9474) (width 0.3556) (layer "F.Cu") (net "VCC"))
 (segment (start 134.6454 97.7112) (end 134.6454 99.1737) (width 0.3556) (layer "F.Cu") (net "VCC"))
 (via (at 133.3246 98.8314) (size 0.6) (drill 0.3) (layers "F.Cu" "B.Cu") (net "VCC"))
 (segment (start 137.2229 99.6309) (end 137.2362 99.6442) (width 0.3556) (layer "B.Cu") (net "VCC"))
 (segment (start 137.2229 98.5266) (end 137.2229 99.6309) (width 0.3556) (layer "B.Cu") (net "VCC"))
 (segment (start 147.1168 96.3118) (end 147.145 96.34) (width 0.1524) (layer "F.Cu") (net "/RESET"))
 (segment (start 142.1282 92.1004) (end 142.1282 93.3856) (width 0.1524) (layer "F.Cu") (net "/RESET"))
 (segment (start 147.1168 94.5388) (end 147.1168 96.3118) (width 0.1524) (layer "F.Cu") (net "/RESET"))
 (segment (start 142.1282 93.3856) (end 142.4178 93.6752) (width 0.1524) (layer "F.Cu") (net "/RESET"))
 (segment (start 142.4178 93.6752) (end 146.2532 93.6752) (width 0.1524) (layer "F.Cu") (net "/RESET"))
 (segment (start 146.2532 93.6752) (end 147.1168 94.5388) (width 0.1524) (layer "F.Cu") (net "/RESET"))
 (segment (start 147.8026 100.1014) (end 149.095 98.809) (width 0.2) (layer "F.Cu") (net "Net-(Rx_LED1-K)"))
 (segment (start 142.3924 100.1014) (end 147.8026 100.1014) (width 0.2) (layer "F.Cu") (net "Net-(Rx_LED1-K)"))
 (segment (start 142.1384 99.3023) (end 142.1384 99.8474) (width 0.2) (layer "F.Cu") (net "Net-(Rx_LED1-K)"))
 (segment (start 142.1384 99.8474) (end 142.3924 100.1014) (width 0.2) (layer "F.Cu") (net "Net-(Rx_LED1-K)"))
 (segment (start 149.095 98.809) (end 149.095 96.34) (width 0.2) (layer "F.Cu") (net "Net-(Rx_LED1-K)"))
 (segment (start 142.1384 98.1573) (end 142.1384 97.0788) (width 0.2032) (layer "F.Cu") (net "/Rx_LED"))
 (via (at 142.1384 97.0788) (size 0.6) (drill 0.3) (layers "F.Cu" "B.Cu") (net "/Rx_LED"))
 (segment (start 139.573 99.6442) (end 142.1384 97.0788) (width 0.2032) (layer "B.Cu") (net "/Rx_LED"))
 (segment (start 138.4312 99.6442) (end 139.573 99.6442) (width 0.2032) (layer "B.Cu") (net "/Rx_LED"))
 (segment (start 140.9192 97.1042) (end 140.9192 97.2058) (width 0.2032) (layer "F.Cu") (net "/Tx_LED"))
 (segment (start 140.9192 97.2058) (end 140.9954 97.282) (width 0.2032) (layer "F.Cu") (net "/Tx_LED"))
 (segment (start 140.9954 97.282) (end 140.9954 98.1573) (width 0.2032) (layer "F.Cu") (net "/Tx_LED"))
 (via (at 140.9192 97.0788) (size 0.6) (drill 0.3) (layers "F.Cu" "B.Cu") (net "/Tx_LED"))
 (segment (start 140.9192 97.1804) (end 139.573 98.5266) (width 0.2032) (layer "B.Cu") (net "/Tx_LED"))
 (segment (start 139.573 98.5266) (end 138.4179 98.5266) (width 0.2032) (layer "B.Cu") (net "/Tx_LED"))
 (segment (start 140.9192 97.1042) (end 140.9192 97.1804) (width 0.2032) (layer "B.Cu") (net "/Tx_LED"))
 (segment (start 133.819 93.13) (end 134.3125 93.13) (width 0.2) (layer "F.Cu") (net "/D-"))
 (segment (start 133.349 93.6) (end 133.819 93.13) (width 0.2) (layer "F.Cu") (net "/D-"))
 (segment (start 132.25 93.6) (end 133.349 93.6) (width 0.2) (layer "F.Cu") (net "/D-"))
 (segment (start 145.845 97.9188) (end 145.845 96.34) (width 0.3556) (layer "F.Cu") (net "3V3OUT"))
 (segment (start 144.3456 98.1202) (end 144.371 98.1456) (width 0.3556) (layer "F.Cu") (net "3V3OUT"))
 (segment (start 144.371 98.1456) (end 145.6182 98.1456) (width 0.3556) (layer "F.Cu") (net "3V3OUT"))
 (segment (start 145.6182 98.1456) (end 145.845 97.9188) (width 0.3556) (layer "F.Cu") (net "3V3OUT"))
 (segment (start 141.7066 100.5332) (end 148.1582 100.5332) (width 0.2) (layer "F.Cu") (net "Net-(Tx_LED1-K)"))
 (segment (start 140.9954 99.822) (end 141.7066 100.5332) (width 0.2) (layer "F.Cu") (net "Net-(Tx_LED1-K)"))
 (segment (start 148.1582 100.5332) (end 149.745 98.9464) (width 0.2) (layer "F.Cu") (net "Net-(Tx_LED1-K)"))
 (segment (start 149.745 98.9464) (end 149.745 96.34) (width 0.2) (layer "F.Cu") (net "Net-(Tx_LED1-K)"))
 (segment (start 140.9954 99.3023) (end 140.9954 99.822) (width 0.2) (layer "F.Cu") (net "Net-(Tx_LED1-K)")))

